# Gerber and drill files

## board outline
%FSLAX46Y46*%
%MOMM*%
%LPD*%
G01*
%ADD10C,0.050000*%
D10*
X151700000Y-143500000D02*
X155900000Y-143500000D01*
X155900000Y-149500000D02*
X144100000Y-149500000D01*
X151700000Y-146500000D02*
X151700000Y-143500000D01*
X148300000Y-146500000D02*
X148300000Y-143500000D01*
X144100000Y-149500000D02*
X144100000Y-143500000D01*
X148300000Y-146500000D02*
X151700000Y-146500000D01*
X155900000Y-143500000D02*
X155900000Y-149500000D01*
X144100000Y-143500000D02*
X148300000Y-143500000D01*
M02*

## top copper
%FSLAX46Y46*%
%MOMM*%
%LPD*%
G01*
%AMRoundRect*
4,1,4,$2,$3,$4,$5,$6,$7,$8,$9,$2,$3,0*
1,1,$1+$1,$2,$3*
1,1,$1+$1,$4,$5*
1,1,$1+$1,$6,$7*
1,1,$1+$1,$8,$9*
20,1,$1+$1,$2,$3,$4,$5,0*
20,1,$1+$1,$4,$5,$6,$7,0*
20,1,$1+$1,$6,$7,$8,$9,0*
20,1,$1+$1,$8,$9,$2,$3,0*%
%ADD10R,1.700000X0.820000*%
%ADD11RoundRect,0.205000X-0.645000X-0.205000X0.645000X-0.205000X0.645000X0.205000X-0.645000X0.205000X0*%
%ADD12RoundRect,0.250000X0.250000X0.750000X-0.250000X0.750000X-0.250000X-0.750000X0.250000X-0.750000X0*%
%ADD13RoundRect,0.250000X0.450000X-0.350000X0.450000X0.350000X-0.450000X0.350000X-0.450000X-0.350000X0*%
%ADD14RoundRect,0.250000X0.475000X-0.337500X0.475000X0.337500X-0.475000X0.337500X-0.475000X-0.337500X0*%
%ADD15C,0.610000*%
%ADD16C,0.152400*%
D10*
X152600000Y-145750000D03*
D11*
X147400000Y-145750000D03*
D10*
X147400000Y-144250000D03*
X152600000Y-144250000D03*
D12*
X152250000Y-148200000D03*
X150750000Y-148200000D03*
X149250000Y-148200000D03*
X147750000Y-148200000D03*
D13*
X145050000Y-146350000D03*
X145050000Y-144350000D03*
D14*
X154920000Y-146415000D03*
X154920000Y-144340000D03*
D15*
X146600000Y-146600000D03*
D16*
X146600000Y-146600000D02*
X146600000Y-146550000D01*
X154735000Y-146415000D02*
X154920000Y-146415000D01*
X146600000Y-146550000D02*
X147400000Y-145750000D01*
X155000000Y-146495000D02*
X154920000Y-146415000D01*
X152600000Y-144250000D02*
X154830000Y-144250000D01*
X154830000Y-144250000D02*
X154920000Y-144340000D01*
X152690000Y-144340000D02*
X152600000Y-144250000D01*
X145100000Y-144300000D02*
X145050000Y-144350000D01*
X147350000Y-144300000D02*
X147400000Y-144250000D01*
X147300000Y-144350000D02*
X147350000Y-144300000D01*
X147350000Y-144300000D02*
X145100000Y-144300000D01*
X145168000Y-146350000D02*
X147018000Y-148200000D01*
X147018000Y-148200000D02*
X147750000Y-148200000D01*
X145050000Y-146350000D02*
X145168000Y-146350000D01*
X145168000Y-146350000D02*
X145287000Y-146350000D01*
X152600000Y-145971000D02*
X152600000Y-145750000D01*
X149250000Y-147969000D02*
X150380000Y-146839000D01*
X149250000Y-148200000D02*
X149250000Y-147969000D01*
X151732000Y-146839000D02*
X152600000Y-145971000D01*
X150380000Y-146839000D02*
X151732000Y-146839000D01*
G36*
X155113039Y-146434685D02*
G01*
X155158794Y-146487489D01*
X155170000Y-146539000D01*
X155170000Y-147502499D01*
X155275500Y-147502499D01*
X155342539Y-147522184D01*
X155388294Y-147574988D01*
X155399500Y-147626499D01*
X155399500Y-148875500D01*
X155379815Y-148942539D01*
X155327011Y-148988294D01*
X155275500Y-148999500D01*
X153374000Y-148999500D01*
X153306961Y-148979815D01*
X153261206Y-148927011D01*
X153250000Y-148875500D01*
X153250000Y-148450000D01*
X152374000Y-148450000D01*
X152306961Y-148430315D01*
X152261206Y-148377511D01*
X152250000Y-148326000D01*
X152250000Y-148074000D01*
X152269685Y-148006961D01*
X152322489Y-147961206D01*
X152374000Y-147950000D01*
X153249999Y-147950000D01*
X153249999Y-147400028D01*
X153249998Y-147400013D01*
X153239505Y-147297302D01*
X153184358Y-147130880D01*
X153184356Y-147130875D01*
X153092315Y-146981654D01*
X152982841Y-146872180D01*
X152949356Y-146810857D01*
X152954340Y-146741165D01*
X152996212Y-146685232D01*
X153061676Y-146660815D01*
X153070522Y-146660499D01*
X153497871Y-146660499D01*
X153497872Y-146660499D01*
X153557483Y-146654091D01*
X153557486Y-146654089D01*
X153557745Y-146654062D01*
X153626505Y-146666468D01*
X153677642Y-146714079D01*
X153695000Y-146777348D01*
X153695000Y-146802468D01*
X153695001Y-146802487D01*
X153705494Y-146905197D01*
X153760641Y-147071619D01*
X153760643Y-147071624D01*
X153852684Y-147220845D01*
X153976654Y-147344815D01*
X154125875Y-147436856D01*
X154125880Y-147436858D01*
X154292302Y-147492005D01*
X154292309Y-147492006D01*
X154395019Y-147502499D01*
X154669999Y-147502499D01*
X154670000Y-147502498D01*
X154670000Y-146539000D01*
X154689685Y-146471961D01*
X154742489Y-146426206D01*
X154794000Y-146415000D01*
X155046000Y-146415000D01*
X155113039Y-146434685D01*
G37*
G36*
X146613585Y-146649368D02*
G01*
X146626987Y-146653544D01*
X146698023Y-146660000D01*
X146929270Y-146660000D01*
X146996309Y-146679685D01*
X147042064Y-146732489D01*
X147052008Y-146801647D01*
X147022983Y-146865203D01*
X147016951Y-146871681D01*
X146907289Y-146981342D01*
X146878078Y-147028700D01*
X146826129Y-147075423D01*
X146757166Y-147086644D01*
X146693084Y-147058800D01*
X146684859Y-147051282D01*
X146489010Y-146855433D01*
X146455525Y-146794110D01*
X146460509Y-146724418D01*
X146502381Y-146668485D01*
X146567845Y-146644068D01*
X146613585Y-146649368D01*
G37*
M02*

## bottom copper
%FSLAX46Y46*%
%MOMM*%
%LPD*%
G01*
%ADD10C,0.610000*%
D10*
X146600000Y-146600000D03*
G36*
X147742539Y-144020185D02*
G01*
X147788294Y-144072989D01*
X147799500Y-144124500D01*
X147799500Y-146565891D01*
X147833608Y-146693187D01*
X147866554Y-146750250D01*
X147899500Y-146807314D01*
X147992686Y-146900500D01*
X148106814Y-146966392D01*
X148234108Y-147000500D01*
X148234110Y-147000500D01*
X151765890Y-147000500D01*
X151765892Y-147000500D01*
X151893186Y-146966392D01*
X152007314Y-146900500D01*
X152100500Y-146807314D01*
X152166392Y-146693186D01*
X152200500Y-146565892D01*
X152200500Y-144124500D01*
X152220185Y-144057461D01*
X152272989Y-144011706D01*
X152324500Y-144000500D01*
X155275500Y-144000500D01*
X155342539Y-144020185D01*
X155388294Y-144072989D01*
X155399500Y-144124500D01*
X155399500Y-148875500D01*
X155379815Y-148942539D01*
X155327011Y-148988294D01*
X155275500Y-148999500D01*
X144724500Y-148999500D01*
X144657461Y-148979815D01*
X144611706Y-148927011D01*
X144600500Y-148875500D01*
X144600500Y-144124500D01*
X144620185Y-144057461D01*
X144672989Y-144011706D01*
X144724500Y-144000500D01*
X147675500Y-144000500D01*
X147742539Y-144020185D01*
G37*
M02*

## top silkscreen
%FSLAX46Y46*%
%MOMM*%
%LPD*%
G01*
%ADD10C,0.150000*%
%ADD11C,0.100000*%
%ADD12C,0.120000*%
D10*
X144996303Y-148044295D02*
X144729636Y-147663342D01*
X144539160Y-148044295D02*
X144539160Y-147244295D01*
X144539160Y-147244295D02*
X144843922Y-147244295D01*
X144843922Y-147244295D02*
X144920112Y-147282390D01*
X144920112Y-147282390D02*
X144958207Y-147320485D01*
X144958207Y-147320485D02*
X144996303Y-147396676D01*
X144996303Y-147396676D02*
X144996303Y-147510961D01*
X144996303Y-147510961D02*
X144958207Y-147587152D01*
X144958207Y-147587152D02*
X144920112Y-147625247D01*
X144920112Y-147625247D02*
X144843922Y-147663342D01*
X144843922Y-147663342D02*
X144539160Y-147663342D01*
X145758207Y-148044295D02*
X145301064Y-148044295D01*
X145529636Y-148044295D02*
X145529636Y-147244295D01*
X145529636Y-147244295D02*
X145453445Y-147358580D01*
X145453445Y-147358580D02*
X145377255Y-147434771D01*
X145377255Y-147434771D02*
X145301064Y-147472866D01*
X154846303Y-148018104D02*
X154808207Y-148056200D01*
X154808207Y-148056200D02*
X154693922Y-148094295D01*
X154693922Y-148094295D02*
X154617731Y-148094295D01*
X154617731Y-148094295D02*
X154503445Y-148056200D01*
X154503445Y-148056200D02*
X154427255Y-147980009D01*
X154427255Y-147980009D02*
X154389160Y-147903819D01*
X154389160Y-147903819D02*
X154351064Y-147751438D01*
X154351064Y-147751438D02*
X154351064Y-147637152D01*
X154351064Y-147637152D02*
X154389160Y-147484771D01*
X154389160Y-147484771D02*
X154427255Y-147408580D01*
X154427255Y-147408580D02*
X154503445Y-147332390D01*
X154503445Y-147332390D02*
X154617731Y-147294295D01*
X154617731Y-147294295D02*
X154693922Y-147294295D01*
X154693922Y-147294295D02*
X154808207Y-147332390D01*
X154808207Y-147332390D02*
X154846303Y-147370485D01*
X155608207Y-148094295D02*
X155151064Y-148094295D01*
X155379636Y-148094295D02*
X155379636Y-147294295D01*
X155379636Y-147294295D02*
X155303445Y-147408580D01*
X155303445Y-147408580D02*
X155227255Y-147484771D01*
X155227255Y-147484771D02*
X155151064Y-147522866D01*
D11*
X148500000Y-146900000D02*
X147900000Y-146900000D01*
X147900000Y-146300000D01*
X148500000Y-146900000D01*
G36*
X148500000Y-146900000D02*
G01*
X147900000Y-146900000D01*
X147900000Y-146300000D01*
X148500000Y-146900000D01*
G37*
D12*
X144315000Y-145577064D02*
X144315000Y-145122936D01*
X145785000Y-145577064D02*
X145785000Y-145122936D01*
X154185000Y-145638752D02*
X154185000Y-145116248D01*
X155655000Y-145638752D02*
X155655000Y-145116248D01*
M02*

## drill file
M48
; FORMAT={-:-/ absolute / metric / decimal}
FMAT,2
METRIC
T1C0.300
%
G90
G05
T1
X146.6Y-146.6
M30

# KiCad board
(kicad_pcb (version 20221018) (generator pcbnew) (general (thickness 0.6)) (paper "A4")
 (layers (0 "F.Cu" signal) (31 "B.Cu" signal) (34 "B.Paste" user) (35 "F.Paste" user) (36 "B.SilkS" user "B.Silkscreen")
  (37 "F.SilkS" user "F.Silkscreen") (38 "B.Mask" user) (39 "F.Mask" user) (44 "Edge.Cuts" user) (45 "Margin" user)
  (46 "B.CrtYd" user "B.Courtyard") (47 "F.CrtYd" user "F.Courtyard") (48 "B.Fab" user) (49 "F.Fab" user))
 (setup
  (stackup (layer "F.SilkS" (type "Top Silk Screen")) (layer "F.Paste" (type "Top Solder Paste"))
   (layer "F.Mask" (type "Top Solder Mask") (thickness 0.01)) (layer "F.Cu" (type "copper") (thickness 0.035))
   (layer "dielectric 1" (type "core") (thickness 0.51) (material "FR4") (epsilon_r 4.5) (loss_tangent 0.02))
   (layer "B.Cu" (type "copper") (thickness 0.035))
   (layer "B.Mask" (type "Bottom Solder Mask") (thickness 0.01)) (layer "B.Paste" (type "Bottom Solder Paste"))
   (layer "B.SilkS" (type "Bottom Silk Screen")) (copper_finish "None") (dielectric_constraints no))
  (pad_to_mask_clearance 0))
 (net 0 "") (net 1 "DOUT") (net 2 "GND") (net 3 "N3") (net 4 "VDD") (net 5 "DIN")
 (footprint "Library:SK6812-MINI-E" (layer "F.Cu") (at 150 145)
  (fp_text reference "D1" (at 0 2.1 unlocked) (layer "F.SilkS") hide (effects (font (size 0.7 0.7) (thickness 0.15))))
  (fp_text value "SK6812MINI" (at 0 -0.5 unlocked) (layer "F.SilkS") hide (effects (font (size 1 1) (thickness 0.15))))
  (fp_poly (pts (xy -1.5 1.9) (xy -2.1 1.9) (xy -2.1 1.3)) (stroke (width 0.1) (type solid)) (fill solid) (layer "F.SilkS"))
  (pad "1" smd rect (at 2.6 0.75) (size 1.7 0.82) (layers "F.Cu" "F.Paste" "F.Mask") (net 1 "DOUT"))
  (pad "2" smd roundrect (at -2.6 0.75) (size 1.7 0.82) (layers "F.Cu" "F.Paste" "F.Mask") (roundrect_rratio 0.25) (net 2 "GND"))
  (pad "3" smd rect (at -2.6 -0.75) (size 1.7 0.82) (layers "F.Cu" "F.Paste" "F.Mask") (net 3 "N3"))
  (pad "4" smd rect (at 2.6 -0.75) (size 1.7 0.82) (layers "F.Cu" "F.Paste" "F.Mask") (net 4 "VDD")))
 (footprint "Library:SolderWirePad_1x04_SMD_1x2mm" (layer "F.Cu") (at 150 148.2 180)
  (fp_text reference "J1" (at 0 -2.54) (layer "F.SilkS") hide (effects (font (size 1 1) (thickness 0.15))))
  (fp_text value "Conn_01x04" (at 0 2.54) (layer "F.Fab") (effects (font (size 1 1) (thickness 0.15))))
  (pad "1" smd roundrect (at -2.25 0 180) (size 1 2) (layers "F.Cu" "F.Paste" "F.Mask") (roundrect_rratio 0.25) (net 2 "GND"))
  (pad "2" smd roundrect (at -0.75 0 180) (size 1 2) (layers "F.Cu" "F.Paste" "F.Mask") (roundrect_rratio 0.25) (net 4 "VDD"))
  (pad "3" smd roundrect (at 0.75 0 180) (size 1 2) (layers "F.Cu" "F.Paste" "F.Mask") (roundrect_rratio 0.25) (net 1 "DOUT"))
  (pad "4" smd roundrect (at 2.25 0 180) (size 1 2) (layers "F.Cu" "F.Paste" "F.Mask") (roundrect_rratio 0.25) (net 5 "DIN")))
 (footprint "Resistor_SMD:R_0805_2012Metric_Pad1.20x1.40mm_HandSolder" (layer "F.Cu") (at 145.05 145.35 90)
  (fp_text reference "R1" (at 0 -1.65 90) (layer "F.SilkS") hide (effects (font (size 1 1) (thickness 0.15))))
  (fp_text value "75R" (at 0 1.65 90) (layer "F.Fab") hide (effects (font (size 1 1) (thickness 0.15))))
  (fp_line (start -0.227064 -0.735) (end 0.227064 -0.735) (stroke (width 0.12) (type solid)) (layer "F.SilkS"))
  (fp_line (start -0.227064 0.735) (end 0.227064 0.735) (stroke (width 0.12) (type solid)) (layer "F.SilkS"))
  (pad "1" smd roundrect (at -1 0 90) (size 1.2 1.4) (layers "F.Cu" "F.Paste" "F.Mask") (roundrect_rratio 0.2083333333) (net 5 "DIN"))
  (pad "2" smd roundrect (at 1 0 90) (size 1.2 1.4) (layers "F.Cu" "F.Paste" "F.Mask") (roundrect_rratio 0.2083333333) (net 3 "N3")))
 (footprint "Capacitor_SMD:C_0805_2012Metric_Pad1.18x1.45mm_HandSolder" (layer "F.Cu") (at 154.92 145.3775 90)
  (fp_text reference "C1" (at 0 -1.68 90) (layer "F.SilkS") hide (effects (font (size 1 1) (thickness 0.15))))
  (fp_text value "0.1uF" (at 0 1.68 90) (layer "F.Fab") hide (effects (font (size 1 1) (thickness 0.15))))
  (fp_line (start -0.261252 -0.735) (end 0.261252 -0.735) (stroke (width 0.12) (type solid)) (layer "F.SilkS"))
  (fp_line (start -0.261252 0.735) (end 0.261252 0.735) (stroke (width 0.12) (type solid)) (layer "F.SilkS"))
  (pad "1" smd roundrect (at -1.0375 0 90) (size 1.175 1.45) (layers "F.Cu" "F.Paste" "F.Mask") (roundrect_rratio 0.2127659574)
   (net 2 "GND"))
  (pad "2" smd roundrect (at 1.0375 0 90) (size 1.175 1.45) (layers "F.Cu" "F.Paste" "F.Mask") (roundrect_rratio 0.2127659574) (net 4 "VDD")))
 (gr_line (start 151.7 143.5) (end 155.9 143.5) (stroke (width 0.05) (type default)) (layer "Edge.Cuts"))
 (gr_line (start 155.9 149.5) (end 144.1 149.5) (stroke (width 0.05) (type default)) (layer "Edge.Cuts"))
 (gr_line (start 151.7 146.5) (end 151.7 143.5) (stroke (width 0.05) (type default)) (layer "Edge.Cuts"))
 (gr_line (start 148.3 146.5) (end 148.3 143.5) (stroke (width 0.05) (type default)) (layer "Edge.Cuts"))
 (gr_line (start 144.1 149.5) (end 144.1 143.5) (stroke (width 0.05) (type default)) (layer "Edge.Cuts"))
 (gr_line (start 148.3 146.5) (end 151.7 146.5) (stroke (width 0.05) (type default)) (layer "Edge.Cuts"))
 (gr_line (start 155.9 143.5) (end 155.9 149.5) (stroke (width 0.05) (type default)) (layer "Edge.Cuts"))
 (gr_line (start 144.1 143.5) (end 148.3 143.5) (stroke (width 0.05) (type default)) (layer "Edge.Cuts"))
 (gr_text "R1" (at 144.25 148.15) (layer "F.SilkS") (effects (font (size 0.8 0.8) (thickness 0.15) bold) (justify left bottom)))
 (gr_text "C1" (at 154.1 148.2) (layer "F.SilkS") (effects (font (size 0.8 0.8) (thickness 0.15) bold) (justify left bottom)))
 (segment (start 146.6 146.6) (end 146.6 146.55) (width 0.1524) (layer "F.Cu") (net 2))
 (segment (start 154.735 146.415) (end 154.92 146.415) (width 0.1524) (layer "F.Cu") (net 2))
 (segment (start 146.6 146.55) (end 147.4 145.75) (width 0.1524) (layer "F.Cu") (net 2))
 (segment (start 155 146.495) (end 154.92 146.415) (width 0.1524) (layer "F.Cu") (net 2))
 (via (at 146.6 146.6) (size 0.61) (drill 0.3) (layers "F.Cu" "B.Cu") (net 2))
 (segment (start 152.6 144.25) (end 154.83 144.25) (width 0.1524) (layer "F.Cu") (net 4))
 (segment (start 154.83 144.25) (end 154.92 144.34) (width 0.1524) (layer "F.Cu") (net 4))
 (segment (start 152.69 144.34) (end 152.6 144.25) (width 0.1524) (layer "F.Cu") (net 4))
 (segment (start 145.1 144.3) (end 145.05 144.35) (width 0.1524) (layer "F.Cu") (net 3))
 (segment (start 147.35 144.3) (end 147.4 144.25) (width 0.1524) (layer "F.Cu") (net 3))
 (segment (start 147.3 144.35) (end 147.35 144.3) (width 0.1524) (layer "F.Cu") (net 3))
 (segment (start 147.35 144.3) (end 145.1 144.3) (width 0.1524) (layer "F.Cu") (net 3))
 (segment (start 145.168 146.35) (end 147.018 148.2) (width 0.1524) (layer "F.Cu") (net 5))
 (segment (start 147.018 148.2) (end 147.75 148.2) (width 0.1524) (layer "F.Cu") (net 5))
 (segment (start 145.05 146.35) (end 145.168 146.35) (width 0.1524) (layer "F.Cu") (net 5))
 (segment (start 145.168 146.35) (end 145.287 146.35) (width 0.1524) (layer "F.Cu") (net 5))
 (segment (start 152.6 145.971) (end 152.6 145.75) (width 0.1524) (layer "F.Cu") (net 1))
 (segment (start 149.25 147.969) (end 150.38 146.839) (width 0.1524) (layer "F.Cu") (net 1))
 (segment (start 149.25 148.2) (end 149.25 147.969) (width 0.1524) (layer "F.Cu") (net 1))
 (segment (start 151.732 146.839) (end 152.6 145.971) (width 0.1524) (layer "F.Cu") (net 1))
 (segment (start 150.38 146.839) (end 151.732 146.839) (width 0.1524) (layer "F.Cu") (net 1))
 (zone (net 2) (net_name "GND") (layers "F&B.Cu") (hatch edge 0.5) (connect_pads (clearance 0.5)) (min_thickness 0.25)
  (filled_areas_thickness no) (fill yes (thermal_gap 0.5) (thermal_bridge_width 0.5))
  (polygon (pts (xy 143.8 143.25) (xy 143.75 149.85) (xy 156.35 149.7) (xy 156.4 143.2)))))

